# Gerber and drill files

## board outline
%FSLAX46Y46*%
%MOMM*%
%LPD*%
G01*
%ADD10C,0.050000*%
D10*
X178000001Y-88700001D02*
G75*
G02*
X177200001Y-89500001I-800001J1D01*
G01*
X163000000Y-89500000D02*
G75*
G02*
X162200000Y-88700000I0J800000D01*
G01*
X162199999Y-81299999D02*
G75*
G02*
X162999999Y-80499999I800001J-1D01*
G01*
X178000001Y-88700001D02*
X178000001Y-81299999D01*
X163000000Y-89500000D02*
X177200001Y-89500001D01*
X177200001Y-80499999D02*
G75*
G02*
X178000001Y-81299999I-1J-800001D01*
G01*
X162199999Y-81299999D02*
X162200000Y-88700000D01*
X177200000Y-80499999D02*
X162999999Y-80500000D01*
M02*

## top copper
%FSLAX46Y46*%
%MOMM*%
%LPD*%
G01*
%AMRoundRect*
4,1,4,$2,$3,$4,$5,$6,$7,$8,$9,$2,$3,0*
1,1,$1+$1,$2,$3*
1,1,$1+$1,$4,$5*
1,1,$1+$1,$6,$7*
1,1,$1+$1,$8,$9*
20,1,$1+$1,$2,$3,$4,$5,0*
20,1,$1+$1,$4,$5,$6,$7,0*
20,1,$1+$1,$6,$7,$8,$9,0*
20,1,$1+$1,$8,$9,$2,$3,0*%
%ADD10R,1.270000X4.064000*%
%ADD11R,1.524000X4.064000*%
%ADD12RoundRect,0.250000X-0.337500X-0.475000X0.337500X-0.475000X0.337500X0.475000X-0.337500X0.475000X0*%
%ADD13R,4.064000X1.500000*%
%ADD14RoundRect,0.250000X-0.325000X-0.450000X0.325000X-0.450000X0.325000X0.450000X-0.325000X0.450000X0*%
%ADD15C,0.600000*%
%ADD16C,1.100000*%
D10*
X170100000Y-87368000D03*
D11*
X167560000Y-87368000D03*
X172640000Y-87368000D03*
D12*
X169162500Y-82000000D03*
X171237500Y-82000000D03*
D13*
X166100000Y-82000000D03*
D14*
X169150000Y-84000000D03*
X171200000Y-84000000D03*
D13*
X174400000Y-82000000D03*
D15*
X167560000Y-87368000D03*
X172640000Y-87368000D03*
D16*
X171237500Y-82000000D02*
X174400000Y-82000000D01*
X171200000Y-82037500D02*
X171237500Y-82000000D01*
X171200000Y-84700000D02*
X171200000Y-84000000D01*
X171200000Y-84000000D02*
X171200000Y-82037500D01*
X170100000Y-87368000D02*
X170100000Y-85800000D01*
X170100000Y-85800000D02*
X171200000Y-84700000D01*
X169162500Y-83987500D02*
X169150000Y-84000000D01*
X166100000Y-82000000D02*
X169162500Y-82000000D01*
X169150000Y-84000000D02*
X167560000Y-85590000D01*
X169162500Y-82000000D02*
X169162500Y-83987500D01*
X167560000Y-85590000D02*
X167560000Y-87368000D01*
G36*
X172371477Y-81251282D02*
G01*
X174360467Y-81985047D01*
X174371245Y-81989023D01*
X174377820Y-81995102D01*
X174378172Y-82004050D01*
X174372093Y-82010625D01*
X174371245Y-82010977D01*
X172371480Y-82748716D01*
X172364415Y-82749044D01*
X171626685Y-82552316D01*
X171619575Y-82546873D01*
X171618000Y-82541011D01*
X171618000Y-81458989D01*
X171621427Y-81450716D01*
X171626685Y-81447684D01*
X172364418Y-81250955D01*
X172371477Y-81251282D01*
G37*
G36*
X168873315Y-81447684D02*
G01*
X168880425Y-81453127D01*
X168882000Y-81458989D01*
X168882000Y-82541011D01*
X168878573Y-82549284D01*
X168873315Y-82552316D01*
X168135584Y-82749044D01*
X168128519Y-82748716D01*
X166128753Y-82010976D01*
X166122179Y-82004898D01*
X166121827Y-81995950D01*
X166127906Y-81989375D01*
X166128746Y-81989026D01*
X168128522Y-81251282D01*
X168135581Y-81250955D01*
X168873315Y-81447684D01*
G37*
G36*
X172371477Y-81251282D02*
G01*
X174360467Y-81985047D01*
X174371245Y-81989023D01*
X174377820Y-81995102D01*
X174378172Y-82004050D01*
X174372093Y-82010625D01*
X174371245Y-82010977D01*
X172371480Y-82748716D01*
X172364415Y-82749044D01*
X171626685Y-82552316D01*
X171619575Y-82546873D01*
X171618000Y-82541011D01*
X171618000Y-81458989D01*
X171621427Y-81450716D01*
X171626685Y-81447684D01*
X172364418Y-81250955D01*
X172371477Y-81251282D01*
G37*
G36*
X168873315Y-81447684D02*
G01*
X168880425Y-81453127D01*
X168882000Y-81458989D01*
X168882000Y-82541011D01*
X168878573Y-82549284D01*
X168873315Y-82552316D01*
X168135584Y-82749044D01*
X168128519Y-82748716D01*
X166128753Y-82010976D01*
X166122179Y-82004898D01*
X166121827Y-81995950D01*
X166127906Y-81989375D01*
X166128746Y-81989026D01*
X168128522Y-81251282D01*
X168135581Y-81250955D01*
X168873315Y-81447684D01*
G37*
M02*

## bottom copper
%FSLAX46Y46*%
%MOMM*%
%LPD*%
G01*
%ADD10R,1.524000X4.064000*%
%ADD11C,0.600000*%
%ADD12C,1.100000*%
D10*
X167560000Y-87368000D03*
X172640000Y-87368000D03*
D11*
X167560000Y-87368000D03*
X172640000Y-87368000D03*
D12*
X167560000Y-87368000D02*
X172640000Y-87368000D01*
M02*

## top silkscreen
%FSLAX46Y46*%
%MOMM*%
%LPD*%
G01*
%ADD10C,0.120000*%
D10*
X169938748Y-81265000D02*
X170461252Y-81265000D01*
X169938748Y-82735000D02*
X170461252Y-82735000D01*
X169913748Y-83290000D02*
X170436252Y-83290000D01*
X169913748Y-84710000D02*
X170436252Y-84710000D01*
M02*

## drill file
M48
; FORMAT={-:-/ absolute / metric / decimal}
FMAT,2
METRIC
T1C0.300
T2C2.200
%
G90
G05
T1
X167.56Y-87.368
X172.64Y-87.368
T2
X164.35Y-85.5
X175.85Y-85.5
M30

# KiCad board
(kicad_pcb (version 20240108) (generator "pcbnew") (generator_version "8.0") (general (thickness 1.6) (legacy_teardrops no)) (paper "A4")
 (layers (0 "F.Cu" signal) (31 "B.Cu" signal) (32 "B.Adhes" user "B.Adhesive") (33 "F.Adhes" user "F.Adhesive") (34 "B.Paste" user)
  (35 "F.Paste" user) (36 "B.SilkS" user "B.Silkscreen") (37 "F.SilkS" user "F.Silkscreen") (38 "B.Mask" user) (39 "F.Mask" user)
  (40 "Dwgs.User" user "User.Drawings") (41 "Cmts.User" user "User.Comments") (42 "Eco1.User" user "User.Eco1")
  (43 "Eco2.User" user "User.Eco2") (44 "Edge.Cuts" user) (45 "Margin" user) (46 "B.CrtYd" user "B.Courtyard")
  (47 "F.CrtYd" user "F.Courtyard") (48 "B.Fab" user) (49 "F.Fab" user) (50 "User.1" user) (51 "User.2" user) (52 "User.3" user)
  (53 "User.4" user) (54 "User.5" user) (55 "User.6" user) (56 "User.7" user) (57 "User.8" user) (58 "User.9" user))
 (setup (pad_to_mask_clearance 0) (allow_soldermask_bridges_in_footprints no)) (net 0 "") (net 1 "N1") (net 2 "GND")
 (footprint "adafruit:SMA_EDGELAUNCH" (layer "F.Cu") (at 170.1 89.4 90)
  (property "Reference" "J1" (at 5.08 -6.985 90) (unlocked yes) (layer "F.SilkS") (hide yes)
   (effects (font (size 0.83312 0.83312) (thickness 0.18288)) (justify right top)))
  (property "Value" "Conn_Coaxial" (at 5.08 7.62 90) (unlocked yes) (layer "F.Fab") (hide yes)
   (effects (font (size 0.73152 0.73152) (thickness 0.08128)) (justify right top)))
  (pad "1" smd rect (at 2.032 0 180) (size 1.27 4.064) (layers "F.Cu" "F.Mask") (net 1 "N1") (solder_mask_margin 0.1016) (zone_connect 2)
   (thermal_bridge_angle 0))
  (pad "2" smd rect (at 2.032 -2.54 180) (size 1.524 4.064) (layers "F.Cu" "F.Mask") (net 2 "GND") (solder_mask_margin 0.1016)
   (thermal_bridge_angle 0))
  (pad "2" smd rect (at 2.032 -2.54 180) (size 1.524 4.064) (layers "B.Cu" "B.Mask") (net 2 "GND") (solder_mask_margin 0.1016)
   (thermal_bridge_angle 0))
  (pad "2" smd rect (at 2.032 2.54 180) (size 1.524 4.064) (layers "F.Cu" "F.Mask") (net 2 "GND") (solder_mask_margin 0.1016)
   (thermal_bridge_angle 0))
  (pad "2" smd rect (at 2.032 2.54 180) (size 1.524 4.064) (layers "B.Cu" "B.Mask") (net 2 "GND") (solder_mask_margin 0.1016)
   (thermal_bridge_angle 0)))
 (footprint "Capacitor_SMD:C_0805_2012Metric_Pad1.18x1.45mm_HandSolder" (layer "F.Cu") (at 170.2 82)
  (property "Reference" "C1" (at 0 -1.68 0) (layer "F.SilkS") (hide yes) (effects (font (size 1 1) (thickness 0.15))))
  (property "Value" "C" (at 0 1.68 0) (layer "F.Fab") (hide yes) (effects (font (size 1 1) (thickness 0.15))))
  (fp_line (start -0.261252 -0.735) (end 0.261252 -0.735) (stroke (width 0.12) (type solid)) (layer "F.SilkS"))
  (fp_line (start -0.261252 0.735) (end 0.261252 0.735) (stroke (width 0.12) (type solid)) (layer "F.SilkS"))
  (pad "1" smd roundrect (at -1.0375 0) (size 1.175 1.45) (layers "F.Cu" "F.Paste" "F.Mask") (roundrect_rratio 0.212766) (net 2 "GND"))
  (pad "2" smd roundrect (at 1.0375 0) (size 1.175 1.45) (layers "F.Cu" "F.Paste" "F.Mask") (roundrect_rratio 0.212766) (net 1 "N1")))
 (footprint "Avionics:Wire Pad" (layer "F.Cu") (at 166.1 82)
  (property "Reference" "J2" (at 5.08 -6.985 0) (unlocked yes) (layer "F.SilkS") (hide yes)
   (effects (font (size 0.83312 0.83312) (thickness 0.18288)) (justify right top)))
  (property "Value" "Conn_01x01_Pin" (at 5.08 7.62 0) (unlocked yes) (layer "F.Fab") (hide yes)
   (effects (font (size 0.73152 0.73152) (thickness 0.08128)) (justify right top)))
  (pad "1" smd rect (at 0 0 90) (size 1.5 4.064) (layers "F.Cu" "F.Mask") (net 2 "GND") (solder_mask_margin 0.1016) (zone_connect 2)
   (thermal_bridge_angle 0)
   (teardrops (best_length_ratio 0.5) (max_length 1) (best_width_ratio 1) (max_width 2) (curve_points 0) (filter_ratio 0.9) (enabled yes)
    (allow_two_segments yes) (prefer_zone_connections yes))))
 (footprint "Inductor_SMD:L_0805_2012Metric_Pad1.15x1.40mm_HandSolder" (layer "F.Cu") (at 170.175 84)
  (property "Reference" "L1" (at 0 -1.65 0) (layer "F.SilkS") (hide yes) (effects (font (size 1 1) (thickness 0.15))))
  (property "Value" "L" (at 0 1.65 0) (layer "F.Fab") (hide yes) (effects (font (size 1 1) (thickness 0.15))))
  (fp_line (start -0.261252 -0.71) (end 0.261252 -0.71) (stroke (width 0.12) (type solid)) (layer "F.SilkS"))
  (fp_line (start -0.261252 0.71) (end 0.261252 0.71) (stroke (width 0.12) (type solid)) (layer "F.SilkS"))
  (pad "1" smd roundrect (at -1.025 0) (size 1.15 1.4) (layers "F.Cu" "F.Paste" "F.Mask") (roundrect_rratio 0.217391) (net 2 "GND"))
  (pad "2" smd roundrect (at 1.025 0) (size 1.15 1.4) (layers "F.Cu" "F.Paste" "F.Mask") (roundrect_rratio 0.217391) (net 1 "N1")))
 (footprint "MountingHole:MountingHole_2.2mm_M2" (layer "F.Cu") (at 175.85 85.5)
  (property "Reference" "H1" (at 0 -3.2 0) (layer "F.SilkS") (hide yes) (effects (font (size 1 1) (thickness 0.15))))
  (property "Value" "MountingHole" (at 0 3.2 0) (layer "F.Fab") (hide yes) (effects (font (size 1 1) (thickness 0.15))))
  (pad "" np_thru_hole circle (at 0 0) (size 2.2 2.2) (drill 2.2) (layers "*.Cu" "*.Mask")))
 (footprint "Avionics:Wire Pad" (layer "F.Cu") (at 174.4 82)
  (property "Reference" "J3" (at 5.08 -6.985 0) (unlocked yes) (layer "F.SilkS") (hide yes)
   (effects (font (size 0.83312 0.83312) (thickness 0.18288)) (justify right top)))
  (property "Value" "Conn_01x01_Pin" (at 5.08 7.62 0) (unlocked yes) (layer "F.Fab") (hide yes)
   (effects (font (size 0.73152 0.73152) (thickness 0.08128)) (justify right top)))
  (pad "1" smd rect (at 0 0 90) (size 1.5 4.064) (layers "F.Cu" "F.Mask") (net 1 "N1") (solder_mask_margin 0.1016) (zone_connect 2)
   (thermal_bridge_angle 0)
   (teardrops (best_length_ratio 0.5) (max_length 1) (best_width_ratio 1) (max_width 2) (curve_points 0) (filter_ratio 0.9) (enabled yes)
    (allow_two_segments yes) (prefer_zone_connections yes))))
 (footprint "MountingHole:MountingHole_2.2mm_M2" (layer "F.Cu") (at 164.35 85.5)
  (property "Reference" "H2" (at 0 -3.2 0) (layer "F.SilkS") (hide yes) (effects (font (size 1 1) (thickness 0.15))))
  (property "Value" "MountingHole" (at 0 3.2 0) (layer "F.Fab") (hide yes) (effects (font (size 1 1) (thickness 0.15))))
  (pad "" np_thru_hole circle (at 0 0) (size 2.2 2.2) (drill 2.2) (layers "*.Cu" "*.Mask")))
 (gr_arc (start 178.000001 88.700001) (mid 177.765686 89.265686) (end 177.200001 89.500001) (stroke (width 0.05) (type default))
  (layer "Edge.Cuts"))
 (gr_arc (start 163 89.5) (mid 162.434315 89.265685) (end 162.2 88.7) (stroke (width 0.05) (type default)) (layer "Edge.Cuts"))
 (gr_arc (start 162.199999 81.299999) (mid 162.434314 80.734314) (end 162.999999 80.499999) (stroke (width 0.05) (type default))
  (layer "Edge.Cuts"))
 (gr_line (start 178.000001 88.700001) (end 178.000001 81.299999) (stroke (width 0.05) (type default)) (layer "Edge.Cuts"))
 (gr_line (start 163 89.5) (end 177.200001 89.500001) (stroke (width 0.05) (type default)) (layer "Edge.Cuts"))
 (gr_arc (start 177.200001 80.499999) (mid 177.765686 80.734314) (end 178.000001 81.299999) (stroke (width 0.05) (type default))
  (layer "Edge.Cuts"))
 (gr_line (start 162.199999 81.299999) (end 162.2 88.7) (stroke (width 0.05) (type default)) (layer "Edge.Cuts"))
 (gr_line (start 177.2 80.499999) (end 162.999999 80.5) (stroke (width 0.05) (type default)) (layer "Edge.Cuts"))
 (segment (start 171.2375 82) (end 174.4 82) (width 1.1) (layer "F.Cu") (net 1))
 (segment (start 171.2 82.0375) (end 171.2375 82) (width 1.1) (layer "F.Cu") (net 1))
 (segment (start 171.2 84.7) (end 171.2 84) (width 1.1) (layer "F.Cu") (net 1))
 (segment (start 171.2 84) (end 171.2 82.0375) (width 1.1) (layer "F.Cu") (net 1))
 (segment (start 170.1 87.368) (end 170.1 85.8) (width 1.1) (layer "F.Cu") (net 1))
 (segment (start 170.1 85.8) (end 171.2 84.7) (width 1.1) (layer "F.Cu") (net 1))
 (segment (start 169.1625 83.9875) (end 169.15 84) (width 1.1) (layer "F.Cu") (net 2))
 (segment (start 166.1 82) (end 169.1625 82) (width 1.1) (layer "F.Cu") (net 2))
 (segment (start 169.15 84) (end 167.56 85.59) (width 1.1) (layer "F.Cu") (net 2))
 (segment (start 169.1625 82) (end 169.1625 83.9875) (width 1.1) (layer "F.Cu") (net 2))
 (segment (start 167.56 85.59) (end 167.56 87.368) (width 1.1) (layer "F.Cu") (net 2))
 (via (at 167.56 87.368) (size 0.6) (drill 0.3) (layers "F.Cu" "B.Cu") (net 2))
 (via (at 172.64 87.368) (size 0.6) (drill 0.3) (layers "F.Cu" "B.Cu") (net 2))
 (segment (start 167.56 87.368) (end 172.64 87.368) (width 1.1) (layer "B.Cu") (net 2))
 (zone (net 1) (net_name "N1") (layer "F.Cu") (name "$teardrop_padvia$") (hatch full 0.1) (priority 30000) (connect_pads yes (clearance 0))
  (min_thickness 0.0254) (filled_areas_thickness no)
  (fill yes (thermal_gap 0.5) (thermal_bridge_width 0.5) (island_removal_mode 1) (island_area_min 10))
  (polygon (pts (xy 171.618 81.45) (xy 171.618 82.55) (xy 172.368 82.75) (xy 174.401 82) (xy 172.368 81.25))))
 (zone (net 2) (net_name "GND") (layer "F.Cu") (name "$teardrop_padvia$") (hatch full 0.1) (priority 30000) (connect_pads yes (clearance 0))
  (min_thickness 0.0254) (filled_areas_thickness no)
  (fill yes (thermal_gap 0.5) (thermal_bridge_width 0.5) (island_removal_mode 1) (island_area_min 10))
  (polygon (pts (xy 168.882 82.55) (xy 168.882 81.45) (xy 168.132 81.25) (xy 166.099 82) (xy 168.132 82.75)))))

